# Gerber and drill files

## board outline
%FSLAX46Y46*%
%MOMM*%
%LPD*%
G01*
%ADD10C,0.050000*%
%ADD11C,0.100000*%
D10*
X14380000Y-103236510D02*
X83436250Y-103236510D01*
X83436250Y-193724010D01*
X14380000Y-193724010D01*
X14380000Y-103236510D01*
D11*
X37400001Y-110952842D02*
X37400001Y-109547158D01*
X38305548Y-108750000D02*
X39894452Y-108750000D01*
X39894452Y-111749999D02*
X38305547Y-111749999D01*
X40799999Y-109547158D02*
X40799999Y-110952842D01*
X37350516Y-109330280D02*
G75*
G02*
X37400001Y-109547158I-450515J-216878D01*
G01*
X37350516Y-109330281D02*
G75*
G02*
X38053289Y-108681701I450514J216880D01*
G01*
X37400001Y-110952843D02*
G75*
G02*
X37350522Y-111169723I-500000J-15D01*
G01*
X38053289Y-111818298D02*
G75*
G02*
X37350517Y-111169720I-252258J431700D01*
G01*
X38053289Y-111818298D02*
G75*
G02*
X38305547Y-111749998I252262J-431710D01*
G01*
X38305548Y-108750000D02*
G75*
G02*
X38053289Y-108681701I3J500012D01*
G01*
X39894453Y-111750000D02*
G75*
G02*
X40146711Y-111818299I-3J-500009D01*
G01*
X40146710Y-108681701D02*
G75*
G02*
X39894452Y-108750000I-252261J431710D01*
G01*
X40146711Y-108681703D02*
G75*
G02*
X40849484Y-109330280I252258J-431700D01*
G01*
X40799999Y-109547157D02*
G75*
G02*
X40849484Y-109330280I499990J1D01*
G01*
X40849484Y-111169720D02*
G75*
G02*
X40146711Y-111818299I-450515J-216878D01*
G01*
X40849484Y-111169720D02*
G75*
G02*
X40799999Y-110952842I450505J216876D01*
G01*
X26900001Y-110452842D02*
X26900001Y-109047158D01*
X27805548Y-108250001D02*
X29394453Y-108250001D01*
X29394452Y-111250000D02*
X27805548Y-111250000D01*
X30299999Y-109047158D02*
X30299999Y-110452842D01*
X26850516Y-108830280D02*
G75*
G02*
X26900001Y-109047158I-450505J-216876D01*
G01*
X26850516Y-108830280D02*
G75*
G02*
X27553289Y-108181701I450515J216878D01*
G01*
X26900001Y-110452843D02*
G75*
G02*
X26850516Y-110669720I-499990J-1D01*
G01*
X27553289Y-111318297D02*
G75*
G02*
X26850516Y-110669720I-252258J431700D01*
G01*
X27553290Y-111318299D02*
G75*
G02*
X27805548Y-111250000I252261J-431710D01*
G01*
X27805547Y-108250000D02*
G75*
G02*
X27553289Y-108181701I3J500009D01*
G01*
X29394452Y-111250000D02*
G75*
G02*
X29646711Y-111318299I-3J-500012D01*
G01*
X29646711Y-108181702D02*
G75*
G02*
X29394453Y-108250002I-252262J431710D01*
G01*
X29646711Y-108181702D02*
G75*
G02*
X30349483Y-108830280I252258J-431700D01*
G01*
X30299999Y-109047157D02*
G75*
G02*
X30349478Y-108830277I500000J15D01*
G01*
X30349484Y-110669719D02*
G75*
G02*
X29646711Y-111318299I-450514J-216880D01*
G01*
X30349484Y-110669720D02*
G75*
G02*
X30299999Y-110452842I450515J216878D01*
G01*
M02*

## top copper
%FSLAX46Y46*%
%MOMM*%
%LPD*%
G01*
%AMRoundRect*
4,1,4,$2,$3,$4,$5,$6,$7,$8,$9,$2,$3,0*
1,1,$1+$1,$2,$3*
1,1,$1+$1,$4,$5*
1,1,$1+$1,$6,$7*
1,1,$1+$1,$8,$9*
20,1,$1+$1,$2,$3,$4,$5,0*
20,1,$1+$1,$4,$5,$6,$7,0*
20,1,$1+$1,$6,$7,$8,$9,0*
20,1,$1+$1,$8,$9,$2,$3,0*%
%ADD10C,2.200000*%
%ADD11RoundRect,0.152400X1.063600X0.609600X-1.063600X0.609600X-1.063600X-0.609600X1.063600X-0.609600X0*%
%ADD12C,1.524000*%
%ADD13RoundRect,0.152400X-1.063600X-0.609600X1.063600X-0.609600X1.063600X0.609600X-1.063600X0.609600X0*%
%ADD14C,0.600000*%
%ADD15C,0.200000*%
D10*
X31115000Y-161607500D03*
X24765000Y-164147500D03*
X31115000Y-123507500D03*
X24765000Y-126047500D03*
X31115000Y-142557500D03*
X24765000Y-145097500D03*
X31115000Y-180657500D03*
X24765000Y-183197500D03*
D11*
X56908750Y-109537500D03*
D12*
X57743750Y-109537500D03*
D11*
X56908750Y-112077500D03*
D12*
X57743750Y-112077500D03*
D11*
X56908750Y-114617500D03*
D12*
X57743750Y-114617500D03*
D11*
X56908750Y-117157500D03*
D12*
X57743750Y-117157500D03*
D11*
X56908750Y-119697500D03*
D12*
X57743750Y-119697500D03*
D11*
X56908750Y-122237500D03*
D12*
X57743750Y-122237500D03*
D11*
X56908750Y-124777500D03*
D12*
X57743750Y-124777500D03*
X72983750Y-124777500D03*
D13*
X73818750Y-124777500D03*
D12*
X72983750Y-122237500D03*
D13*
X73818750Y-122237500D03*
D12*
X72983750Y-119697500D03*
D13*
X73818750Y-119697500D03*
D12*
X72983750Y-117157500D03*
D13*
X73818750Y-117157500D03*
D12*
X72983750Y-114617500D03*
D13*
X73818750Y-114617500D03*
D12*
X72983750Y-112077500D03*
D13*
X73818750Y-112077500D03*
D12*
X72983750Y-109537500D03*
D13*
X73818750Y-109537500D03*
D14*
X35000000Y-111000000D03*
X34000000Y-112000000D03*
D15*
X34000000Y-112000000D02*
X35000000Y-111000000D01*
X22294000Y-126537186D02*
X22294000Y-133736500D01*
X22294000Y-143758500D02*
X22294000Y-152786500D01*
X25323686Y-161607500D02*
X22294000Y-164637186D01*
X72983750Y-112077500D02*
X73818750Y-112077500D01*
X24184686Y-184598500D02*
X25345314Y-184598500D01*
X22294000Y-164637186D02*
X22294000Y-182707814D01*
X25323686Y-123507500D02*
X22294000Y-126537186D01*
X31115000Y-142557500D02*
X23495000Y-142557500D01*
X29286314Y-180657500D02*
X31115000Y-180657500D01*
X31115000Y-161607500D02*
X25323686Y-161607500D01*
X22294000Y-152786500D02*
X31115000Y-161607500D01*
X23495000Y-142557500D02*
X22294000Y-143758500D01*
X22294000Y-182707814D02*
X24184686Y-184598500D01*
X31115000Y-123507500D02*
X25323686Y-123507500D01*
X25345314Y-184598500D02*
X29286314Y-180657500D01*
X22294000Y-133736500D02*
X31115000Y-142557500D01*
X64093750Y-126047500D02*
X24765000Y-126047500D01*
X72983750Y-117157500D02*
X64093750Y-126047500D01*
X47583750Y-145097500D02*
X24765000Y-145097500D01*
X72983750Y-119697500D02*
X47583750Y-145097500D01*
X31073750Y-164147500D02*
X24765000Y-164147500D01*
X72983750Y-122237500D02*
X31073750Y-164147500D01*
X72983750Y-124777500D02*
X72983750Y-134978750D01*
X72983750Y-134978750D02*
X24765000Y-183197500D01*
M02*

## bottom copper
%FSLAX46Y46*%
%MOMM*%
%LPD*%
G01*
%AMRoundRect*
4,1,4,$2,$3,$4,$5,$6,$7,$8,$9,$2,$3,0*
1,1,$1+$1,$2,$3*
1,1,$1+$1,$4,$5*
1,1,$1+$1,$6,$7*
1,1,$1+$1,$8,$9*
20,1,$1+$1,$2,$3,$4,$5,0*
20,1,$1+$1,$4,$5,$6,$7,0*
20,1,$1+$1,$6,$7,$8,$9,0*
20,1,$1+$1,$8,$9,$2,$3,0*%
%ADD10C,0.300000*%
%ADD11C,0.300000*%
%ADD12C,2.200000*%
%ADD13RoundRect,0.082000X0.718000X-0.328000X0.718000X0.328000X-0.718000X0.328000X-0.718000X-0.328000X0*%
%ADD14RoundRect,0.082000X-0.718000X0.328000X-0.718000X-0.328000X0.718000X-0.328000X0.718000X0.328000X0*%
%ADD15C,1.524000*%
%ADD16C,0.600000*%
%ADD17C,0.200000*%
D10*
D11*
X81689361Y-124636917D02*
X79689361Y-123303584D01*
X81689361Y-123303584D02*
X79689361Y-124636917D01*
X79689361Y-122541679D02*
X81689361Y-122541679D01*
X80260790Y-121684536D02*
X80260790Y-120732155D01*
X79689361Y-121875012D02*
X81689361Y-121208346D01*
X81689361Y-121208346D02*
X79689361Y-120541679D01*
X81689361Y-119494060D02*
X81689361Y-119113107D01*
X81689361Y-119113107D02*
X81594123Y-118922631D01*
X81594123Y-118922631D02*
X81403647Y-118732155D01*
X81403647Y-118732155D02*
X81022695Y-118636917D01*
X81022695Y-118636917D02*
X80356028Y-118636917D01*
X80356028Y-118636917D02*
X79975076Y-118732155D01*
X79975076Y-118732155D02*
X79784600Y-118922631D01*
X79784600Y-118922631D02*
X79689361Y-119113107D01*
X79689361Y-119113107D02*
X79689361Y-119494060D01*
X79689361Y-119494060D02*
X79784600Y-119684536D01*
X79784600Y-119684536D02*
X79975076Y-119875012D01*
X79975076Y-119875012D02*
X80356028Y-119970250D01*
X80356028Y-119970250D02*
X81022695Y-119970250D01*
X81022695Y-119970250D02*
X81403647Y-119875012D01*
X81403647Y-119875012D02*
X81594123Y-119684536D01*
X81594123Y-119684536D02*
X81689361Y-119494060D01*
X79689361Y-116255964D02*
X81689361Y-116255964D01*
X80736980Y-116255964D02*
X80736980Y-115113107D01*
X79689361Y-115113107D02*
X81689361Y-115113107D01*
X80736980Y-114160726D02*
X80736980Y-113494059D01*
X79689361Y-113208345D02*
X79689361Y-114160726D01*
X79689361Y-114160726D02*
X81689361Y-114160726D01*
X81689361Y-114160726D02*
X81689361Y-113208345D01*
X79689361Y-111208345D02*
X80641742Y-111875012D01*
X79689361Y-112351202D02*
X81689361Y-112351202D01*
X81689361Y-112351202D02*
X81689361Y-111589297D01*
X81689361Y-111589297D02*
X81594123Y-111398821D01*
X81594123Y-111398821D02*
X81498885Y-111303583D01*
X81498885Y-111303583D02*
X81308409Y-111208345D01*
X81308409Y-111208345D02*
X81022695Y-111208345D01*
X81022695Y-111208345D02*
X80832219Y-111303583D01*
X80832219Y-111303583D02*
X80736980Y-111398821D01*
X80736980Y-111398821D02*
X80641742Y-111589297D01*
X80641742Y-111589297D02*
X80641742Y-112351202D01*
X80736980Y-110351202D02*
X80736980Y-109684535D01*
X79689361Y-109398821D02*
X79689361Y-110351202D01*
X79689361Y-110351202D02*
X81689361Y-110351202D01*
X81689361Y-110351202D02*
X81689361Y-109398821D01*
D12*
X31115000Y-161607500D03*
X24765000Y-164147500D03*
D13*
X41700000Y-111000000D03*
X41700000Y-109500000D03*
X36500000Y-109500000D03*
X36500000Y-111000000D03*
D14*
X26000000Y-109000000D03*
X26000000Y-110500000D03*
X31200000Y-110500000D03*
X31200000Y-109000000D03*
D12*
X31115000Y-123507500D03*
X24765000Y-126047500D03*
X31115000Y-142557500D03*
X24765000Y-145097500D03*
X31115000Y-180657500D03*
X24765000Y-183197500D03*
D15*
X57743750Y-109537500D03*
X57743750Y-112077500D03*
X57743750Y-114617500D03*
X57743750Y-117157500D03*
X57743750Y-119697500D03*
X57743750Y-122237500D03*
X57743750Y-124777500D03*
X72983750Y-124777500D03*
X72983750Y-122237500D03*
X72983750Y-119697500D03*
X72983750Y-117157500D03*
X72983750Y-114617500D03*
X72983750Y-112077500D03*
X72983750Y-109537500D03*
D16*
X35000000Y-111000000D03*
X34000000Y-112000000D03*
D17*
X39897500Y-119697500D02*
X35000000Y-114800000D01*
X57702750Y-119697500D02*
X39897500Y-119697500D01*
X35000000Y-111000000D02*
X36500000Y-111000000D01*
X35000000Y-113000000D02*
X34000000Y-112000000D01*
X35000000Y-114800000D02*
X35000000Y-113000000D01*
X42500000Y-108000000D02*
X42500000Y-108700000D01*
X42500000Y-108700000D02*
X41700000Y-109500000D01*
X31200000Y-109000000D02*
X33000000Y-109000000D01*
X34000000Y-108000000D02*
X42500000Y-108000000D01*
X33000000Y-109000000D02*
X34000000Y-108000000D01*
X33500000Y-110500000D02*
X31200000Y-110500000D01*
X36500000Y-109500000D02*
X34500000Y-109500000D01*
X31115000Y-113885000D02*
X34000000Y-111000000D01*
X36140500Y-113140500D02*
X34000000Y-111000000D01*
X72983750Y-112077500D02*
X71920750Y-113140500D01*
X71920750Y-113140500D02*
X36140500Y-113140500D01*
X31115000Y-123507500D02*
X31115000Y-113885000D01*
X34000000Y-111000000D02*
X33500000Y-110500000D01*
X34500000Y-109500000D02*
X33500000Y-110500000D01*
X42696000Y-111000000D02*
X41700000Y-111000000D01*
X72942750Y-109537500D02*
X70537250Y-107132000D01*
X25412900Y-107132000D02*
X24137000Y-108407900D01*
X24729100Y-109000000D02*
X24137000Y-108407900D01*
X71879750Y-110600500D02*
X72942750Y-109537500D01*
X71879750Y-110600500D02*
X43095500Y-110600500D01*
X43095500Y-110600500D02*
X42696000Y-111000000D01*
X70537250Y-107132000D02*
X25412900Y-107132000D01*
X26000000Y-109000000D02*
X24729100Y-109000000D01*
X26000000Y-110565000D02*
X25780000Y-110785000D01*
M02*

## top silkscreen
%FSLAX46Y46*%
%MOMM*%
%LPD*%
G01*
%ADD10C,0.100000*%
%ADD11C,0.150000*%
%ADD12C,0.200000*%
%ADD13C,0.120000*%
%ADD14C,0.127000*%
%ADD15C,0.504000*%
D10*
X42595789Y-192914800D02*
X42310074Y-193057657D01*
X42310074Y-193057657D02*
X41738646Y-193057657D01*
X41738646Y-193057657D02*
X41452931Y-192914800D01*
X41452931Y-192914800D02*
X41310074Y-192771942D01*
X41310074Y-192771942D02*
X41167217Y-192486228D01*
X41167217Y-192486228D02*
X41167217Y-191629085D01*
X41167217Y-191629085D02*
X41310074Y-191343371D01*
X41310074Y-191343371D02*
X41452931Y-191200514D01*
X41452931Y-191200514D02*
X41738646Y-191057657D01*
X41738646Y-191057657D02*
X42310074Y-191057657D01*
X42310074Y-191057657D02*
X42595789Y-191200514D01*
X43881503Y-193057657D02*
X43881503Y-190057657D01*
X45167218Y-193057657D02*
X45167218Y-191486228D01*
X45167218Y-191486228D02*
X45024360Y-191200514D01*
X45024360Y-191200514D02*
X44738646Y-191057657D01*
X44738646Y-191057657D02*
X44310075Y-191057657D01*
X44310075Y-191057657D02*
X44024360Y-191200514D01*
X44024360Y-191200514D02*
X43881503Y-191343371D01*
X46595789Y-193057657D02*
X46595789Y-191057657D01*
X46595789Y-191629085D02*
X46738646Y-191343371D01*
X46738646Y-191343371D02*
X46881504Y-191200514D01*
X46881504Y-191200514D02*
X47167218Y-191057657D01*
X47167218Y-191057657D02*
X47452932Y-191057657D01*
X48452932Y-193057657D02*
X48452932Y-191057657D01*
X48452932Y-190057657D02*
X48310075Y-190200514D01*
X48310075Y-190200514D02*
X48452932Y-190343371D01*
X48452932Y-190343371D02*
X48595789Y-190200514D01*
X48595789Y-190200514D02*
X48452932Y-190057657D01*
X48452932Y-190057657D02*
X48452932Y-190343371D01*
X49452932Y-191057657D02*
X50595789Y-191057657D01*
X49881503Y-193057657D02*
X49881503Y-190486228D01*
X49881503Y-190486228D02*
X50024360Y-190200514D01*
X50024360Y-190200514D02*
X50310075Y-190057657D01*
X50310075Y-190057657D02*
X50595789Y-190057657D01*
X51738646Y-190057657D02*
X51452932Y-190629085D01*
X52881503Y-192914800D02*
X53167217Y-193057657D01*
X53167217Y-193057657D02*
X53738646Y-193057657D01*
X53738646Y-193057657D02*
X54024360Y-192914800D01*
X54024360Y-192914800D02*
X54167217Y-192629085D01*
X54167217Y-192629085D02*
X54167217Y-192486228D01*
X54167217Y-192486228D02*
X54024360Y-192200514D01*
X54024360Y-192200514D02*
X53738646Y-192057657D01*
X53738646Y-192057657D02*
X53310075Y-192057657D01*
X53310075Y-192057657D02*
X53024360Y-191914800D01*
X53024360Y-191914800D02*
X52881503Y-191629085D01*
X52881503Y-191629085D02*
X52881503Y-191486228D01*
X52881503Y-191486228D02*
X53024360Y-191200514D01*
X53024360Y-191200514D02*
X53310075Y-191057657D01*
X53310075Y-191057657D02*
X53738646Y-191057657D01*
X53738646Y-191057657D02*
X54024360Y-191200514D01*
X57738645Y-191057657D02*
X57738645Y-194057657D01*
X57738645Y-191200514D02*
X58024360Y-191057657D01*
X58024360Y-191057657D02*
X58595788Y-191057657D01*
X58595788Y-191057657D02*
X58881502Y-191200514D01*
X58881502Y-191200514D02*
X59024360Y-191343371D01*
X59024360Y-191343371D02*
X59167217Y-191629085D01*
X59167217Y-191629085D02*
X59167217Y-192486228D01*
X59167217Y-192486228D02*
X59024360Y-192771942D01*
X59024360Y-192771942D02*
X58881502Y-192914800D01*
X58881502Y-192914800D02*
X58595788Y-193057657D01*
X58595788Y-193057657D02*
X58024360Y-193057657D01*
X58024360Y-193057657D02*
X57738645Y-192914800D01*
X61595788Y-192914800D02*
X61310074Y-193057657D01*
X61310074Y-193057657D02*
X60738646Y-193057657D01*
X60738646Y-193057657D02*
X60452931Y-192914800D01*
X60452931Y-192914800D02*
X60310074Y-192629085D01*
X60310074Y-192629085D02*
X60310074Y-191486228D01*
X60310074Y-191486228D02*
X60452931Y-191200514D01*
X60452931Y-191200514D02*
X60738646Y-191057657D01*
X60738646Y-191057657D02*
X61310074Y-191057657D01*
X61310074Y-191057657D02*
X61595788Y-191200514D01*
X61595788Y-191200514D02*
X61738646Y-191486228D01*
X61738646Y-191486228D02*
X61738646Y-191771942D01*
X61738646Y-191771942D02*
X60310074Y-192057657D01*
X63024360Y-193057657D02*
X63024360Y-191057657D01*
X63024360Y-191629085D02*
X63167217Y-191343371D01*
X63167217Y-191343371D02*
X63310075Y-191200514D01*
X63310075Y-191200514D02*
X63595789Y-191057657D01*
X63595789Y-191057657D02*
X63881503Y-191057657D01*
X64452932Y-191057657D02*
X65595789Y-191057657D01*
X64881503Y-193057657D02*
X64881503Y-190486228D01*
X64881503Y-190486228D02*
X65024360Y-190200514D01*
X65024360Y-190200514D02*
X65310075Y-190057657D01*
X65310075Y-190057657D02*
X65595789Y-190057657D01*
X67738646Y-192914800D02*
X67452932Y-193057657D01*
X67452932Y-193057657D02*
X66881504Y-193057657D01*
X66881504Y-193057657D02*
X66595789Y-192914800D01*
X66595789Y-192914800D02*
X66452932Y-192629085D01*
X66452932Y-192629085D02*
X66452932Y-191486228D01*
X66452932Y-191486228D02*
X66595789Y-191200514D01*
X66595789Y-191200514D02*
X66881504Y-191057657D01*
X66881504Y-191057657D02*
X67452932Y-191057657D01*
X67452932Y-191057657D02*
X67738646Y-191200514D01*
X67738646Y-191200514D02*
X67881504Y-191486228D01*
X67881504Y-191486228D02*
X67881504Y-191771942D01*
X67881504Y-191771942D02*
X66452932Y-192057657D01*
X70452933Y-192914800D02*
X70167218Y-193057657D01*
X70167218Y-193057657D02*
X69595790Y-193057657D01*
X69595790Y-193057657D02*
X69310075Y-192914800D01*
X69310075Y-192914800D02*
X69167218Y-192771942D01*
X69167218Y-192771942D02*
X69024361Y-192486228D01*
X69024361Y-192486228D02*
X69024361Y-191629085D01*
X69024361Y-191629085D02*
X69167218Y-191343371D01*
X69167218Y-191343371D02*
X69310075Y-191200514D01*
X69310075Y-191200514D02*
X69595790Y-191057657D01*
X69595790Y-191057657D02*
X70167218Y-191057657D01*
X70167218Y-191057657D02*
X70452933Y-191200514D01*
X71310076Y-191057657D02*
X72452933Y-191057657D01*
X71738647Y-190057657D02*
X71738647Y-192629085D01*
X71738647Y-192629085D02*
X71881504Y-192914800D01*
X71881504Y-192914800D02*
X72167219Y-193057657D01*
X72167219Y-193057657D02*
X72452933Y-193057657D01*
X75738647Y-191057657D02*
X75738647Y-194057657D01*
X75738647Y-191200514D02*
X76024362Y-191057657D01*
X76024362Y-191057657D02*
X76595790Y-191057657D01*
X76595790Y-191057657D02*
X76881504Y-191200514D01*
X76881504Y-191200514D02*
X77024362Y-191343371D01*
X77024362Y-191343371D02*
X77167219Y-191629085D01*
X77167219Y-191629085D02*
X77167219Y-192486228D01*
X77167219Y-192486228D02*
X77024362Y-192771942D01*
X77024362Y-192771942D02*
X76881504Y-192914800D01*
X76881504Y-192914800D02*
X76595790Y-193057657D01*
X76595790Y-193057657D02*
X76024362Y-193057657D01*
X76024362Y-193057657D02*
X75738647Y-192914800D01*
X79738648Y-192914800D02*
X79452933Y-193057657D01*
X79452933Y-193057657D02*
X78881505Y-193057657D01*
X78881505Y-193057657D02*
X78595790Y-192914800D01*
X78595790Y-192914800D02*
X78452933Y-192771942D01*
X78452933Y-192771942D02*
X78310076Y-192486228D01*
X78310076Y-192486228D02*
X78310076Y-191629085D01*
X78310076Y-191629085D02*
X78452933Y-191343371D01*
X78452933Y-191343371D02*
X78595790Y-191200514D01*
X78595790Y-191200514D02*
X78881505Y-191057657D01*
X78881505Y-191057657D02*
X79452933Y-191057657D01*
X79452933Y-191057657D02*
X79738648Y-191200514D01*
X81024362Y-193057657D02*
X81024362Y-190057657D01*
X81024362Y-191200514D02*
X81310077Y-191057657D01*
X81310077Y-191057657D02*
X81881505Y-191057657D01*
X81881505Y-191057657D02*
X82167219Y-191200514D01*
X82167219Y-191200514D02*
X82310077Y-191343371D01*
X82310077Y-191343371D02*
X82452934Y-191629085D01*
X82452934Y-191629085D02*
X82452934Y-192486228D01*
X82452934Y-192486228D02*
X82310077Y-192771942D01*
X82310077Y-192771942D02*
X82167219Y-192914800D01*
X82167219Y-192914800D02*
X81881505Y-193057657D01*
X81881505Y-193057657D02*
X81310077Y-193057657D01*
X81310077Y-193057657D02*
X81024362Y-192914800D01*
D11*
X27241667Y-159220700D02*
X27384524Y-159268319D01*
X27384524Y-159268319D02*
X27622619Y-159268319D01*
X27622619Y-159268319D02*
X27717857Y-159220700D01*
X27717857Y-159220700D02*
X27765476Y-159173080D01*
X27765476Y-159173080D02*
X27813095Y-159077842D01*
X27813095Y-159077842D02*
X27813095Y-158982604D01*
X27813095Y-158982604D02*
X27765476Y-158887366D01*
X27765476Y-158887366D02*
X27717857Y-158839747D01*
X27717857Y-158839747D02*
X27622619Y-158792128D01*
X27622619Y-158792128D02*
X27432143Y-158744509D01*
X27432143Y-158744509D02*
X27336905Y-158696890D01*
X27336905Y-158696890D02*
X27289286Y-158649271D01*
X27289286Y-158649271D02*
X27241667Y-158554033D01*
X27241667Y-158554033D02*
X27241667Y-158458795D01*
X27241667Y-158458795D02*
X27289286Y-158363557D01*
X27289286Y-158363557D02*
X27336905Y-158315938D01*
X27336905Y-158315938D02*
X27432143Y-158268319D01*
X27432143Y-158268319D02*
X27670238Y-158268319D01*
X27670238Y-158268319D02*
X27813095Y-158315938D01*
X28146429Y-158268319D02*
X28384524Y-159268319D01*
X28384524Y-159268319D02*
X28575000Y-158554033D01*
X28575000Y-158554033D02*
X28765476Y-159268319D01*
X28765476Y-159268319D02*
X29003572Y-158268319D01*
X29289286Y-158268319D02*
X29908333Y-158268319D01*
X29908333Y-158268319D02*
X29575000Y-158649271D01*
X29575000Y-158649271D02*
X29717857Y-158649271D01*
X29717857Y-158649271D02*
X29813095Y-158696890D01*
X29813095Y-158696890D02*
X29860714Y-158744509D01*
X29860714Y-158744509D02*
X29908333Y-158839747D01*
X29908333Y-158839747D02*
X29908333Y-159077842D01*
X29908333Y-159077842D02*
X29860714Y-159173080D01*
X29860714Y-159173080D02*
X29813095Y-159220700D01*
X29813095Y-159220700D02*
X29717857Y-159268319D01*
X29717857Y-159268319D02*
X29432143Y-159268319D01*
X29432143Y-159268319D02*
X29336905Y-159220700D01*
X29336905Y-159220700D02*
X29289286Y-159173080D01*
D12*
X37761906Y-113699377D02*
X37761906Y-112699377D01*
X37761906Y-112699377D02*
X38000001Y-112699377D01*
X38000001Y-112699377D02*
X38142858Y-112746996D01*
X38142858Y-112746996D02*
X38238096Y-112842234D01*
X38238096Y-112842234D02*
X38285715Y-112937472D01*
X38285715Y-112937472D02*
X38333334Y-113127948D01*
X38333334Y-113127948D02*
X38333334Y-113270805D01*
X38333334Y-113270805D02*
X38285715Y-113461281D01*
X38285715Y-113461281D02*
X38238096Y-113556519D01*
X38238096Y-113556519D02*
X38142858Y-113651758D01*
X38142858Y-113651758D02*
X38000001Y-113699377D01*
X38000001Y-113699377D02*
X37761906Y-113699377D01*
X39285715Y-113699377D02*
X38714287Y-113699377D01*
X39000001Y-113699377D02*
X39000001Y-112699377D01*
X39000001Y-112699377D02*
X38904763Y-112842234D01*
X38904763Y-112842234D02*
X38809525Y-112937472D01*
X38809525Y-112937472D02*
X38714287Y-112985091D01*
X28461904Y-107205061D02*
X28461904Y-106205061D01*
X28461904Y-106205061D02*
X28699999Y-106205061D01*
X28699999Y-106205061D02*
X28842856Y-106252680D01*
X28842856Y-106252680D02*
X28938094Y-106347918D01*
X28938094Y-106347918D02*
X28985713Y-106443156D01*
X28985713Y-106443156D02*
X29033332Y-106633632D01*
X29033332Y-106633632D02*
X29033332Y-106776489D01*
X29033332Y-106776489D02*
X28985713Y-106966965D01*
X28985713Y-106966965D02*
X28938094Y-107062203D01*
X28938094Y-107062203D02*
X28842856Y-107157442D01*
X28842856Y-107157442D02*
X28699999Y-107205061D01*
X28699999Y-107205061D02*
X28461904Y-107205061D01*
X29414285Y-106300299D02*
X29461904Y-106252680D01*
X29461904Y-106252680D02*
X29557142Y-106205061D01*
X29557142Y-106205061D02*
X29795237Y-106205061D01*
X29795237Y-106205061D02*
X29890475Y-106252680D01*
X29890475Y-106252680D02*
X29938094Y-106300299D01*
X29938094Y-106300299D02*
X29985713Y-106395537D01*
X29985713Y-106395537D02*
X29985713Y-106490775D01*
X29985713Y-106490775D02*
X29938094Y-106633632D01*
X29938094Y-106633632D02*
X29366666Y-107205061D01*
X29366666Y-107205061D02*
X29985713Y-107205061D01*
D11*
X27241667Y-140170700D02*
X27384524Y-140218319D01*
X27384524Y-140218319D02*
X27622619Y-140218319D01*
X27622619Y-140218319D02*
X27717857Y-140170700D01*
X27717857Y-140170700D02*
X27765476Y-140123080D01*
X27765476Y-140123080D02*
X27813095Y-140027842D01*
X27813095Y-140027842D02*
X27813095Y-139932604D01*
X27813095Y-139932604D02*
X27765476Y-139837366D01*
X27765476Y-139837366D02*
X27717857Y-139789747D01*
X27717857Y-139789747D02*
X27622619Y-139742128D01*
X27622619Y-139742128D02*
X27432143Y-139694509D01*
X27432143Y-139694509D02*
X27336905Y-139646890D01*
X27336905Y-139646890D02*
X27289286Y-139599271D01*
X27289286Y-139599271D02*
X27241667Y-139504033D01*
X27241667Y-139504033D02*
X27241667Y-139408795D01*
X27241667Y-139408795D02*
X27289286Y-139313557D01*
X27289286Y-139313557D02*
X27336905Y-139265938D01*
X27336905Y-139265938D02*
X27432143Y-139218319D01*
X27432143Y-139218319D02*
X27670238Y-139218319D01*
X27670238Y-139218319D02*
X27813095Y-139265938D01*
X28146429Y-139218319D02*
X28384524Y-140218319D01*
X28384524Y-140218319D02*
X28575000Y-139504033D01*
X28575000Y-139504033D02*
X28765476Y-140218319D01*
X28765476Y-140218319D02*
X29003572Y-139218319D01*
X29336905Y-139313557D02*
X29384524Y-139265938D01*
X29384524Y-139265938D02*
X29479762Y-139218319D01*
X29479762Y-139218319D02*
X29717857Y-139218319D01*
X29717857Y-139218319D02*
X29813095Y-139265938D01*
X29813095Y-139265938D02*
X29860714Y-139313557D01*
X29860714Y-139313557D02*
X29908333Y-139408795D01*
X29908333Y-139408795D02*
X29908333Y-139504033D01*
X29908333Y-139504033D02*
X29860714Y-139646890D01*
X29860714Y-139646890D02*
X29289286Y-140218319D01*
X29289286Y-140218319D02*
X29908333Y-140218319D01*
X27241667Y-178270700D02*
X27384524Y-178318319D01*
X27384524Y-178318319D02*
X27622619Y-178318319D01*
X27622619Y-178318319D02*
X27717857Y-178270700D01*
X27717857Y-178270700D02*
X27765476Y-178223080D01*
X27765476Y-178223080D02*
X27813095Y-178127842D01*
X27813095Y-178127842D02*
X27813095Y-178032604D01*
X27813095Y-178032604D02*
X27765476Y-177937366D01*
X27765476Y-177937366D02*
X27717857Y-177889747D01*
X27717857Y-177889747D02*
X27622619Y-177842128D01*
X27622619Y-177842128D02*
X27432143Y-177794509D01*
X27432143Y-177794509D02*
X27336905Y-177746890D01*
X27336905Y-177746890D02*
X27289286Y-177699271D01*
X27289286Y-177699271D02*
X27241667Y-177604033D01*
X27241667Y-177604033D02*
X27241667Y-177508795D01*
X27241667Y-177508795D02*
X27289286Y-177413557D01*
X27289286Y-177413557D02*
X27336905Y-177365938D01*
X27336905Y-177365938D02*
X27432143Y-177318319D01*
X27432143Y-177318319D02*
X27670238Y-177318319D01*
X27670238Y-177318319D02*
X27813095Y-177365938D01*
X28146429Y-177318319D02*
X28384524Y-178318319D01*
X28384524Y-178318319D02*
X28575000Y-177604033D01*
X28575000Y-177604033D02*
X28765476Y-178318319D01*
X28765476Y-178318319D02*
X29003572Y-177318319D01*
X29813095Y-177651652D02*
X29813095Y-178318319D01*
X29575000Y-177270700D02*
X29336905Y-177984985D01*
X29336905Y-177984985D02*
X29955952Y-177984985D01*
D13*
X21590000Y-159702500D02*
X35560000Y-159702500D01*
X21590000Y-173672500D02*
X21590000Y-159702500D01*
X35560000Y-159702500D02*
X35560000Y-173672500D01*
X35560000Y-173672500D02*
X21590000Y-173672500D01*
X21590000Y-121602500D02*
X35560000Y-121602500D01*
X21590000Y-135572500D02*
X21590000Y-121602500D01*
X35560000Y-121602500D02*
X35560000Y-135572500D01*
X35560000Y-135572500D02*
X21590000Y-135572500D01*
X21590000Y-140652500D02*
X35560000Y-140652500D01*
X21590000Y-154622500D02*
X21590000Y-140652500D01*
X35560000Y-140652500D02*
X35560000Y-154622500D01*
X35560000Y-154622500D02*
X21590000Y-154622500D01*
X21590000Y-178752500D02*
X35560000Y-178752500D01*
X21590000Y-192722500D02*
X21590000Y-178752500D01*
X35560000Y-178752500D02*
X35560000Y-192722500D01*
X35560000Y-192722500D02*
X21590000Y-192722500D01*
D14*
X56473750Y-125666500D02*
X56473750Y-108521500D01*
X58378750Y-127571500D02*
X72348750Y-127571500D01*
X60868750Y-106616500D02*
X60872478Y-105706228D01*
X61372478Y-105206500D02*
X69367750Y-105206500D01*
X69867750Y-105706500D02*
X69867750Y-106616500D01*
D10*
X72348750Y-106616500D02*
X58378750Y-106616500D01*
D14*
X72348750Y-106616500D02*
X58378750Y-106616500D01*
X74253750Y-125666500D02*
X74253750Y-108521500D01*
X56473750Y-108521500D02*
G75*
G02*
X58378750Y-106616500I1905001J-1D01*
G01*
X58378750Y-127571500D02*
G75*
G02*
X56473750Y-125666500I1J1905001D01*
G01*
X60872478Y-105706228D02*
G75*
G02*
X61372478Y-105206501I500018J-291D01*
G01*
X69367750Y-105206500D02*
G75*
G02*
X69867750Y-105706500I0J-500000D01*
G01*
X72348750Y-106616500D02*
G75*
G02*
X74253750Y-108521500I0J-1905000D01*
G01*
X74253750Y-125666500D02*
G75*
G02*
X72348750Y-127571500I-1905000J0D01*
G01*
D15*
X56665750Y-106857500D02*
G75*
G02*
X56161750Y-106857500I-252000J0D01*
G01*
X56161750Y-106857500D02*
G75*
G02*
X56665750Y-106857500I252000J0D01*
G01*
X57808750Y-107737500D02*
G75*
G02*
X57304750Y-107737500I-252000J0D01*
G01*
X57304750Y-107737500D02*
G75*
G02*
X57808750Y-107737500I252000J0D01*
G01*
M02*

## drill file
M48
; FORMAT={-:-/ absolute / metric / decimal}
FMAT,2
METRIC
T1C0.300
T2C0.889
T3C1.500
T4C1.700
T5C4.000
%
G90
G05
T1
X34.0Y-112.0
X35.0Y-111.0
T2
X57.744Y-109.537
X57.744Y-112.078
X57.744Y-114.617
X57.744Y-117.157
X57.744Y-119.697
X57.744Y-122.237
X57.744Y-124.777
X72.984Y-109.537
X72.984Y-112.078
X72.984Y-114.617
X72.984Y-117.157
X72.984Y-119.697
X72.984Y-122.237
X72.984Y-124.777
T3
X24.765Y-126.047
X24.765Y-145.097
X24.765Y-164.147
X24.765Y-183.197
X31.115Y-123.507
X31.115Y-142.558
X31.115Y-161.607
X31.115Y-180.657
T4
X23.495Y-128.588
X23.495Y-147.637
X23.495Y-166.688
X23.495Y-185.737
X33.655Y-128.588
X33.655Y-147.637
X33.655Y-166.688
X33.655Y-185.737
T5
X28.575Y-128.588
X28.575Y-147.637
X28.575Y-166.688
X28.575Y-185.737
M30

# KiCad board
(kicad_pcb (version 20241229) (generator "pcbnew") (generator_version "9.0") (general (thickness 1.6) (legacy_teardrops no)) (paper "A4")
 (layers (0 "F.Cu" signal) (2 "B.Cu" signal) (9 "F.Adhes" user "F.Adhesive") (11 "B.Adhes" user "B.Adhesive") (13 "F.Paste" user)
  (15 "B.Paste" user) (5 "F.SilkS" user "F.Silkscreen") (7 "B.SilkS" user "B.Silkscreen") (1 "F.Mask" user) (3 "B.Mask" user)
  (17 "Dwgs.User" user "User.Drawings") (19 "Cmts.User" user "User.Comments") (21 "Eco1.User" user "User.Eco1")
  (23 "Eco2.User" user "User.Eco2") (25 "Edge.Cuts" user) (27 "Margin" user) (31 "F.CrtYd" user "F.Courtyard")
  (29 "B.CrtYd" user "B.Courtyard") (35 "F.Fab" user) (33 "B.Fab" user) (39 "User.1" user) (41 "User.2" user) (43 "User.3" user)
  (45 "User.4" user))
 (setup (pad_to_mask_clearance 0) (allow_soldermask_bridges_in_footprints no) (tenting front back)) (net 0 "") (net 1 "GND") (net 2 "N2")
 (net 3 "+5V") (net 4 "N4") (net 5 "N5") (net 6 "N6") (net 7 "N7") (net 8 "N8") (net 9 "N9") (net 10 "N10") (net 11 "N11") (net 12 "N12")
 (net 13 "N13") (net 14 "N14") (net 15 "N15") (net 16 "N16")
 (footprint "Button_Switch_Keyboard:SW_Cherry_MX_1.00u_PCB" (layer "F.Cu") (at 31.115 161.6075)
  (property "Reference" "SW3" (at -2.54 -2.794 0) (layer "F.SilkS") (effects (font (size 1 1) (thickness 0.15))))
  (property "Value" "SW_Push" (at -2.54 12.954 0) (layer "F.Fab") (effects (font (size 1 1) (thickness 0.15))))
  (fp_line (start -9.525 -1.905) (end 4.445 -1.905) (stroke (width 0.12) (type solid)) (layer "F.SilkS"))
  (fp_line (start -9.525 12.065) (end -9.525 -1.905) (stroke (width 0.12) (type solid)) (layer "F.SilkS"))
  (fp_line (start 4.445 -1.905) (end 4.445 12.065) (stroke (width 0.12) (type solid)) (layer "F.SilkS"))
  (fp_line (start 4.445 12.065) (end -9.525 12.065) (stroke (width 0.12) (type solid)) (layer "F.SilkS"))
  (pad "" np_thru_hole circle (at -7.62 5.08) (size 1.7 1.7) (drill 1.7) (layers "*.Cu" "*.Mask"))
  (pad "" np_thru_hole circle (at -2.54 5.08) (size 4 4) (drill 4) (layers "*.Cu" "*.Mask"))
  (pad "" np_thru_hole circle (at 2.54 5.08) (size 1.7 1.7) (drill 1.7) (layers "*.Cu" "*.Mask"))
  (pad "1" thru_hole circle (at 0 0) (size 2.2 2.2) (drill 1.5) (layers "*.Cu" "*.Mask") (remove_unused_layers no) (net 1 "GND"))
  (pad "2" thru_hole circle (at -6.35 2.54) (size 2.2 2.2) (drill 1.5) (layers "*.Cu" "*.Mask") (remove_unused_layers no) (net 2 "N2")))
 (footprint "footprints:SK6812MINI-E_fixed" (layer "F.Cu") (at 39.100001 110.147158 180)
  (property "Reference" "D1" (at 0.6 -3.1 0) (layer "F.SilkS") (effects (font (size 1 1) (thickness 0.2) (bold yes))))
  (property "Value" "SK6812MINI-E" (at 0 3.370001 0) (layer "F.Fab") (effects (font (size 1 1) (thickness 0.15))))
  (fp_line (start 1.7 -0.805684) (end 1.7 0.6) (stroke (width 0.1) (type solid)) (layer "Edge.Cuts"))
  (fp_line (start 0.794453 1.397158) (end -0.794451 1.397158) (stroke (width 0.1) (type solid)) (layer "Edge.Cuts"))
  (fp_line (start -0.794451 -1.602841) (end 0.794454 -1.602841) (stroke (width 0.1) (type solid)) (layer "Edge.Cuts"))
  (fp_line (start -1.699998 0.6) (end -1.699998 -0.805684) (stroke (width 0.1) (type solid)) (layer "Edge.Cuts"))
  (fp_arc (start 1.749485 0.816878) (mid 1.712528 0.711226) (end 1.7 0.6) (stroke (width 0.1) (type solid)) (layer "Edge.Cuts"))
  (fp_arc (start 1.749485 0.816877) (mid 1.638073 1.401193) (end 1.046712 1.465457) (stroke (width 0.1) (type solid)) (layer "Edge.Cuts"))
  (fp_arc (start 1.7 -0.805685) (mid 1.712528 -0.91691) (end 1.749485 -1.022562) (stroke (width 0.1) (type solid)) (layer "Edge.Cuts"))
  (fp_arc (start 1.046712 -1.67114) (mid 1.638072 -1.606876) (end 1.749485 -1.022562) (stroke (width 0.1) (type solid)) (layer "Edge.Cuts"))
  (fp_arc (start 1.046712 -1.67114) (mid 0.925124 -1.620218) (end 0.794454 -1.602841) (stroke (width 0.1) (type solid)) (layer "Edge.Cuts"))
  (fp_arc (start 0.794453 1.397158) (mid 0.925124 1.414535) (end 1.046712 1.465457) (stroke (width 0.1) (type solid)) (layer "Edge.Cuts"))
  (fp_arc (start -0.794452 -1.602842) (mid -0.925122 -1.620219) (end -1.04671 -1.671141) (stroke (width 0.1) (type solid))
   (layer "Edge.Cuts"))
  (fp_arc (start -1.046709 1.465457) (mid -0.925121 1.414535) (end -0.794451 1.397158) (stroke (width 0.1) (type solid)) (layer "Edge.Cuts"))
  (fp_arc (start -1.04671 1.465455) (mid -1.638069 1.401192) (end -1.749483 0.816878) (stroke (width 0.1) (type solid)) (layer "Edge.Cuts"))
  (fp_arc (start -1.699998 0.600001) (mid -1.712526 0.711226) (end -1.749483 0.816878) (stroke (width 0.1) (type solid)) (layer "Edge.Cuts"))
  (fp_arc (start -1.749483 -1.022562) (mid -1.63807 -1.606877) (end -1.04671 -1.671141) (stroke (width 0.1) (type solid))
   (layer "Edge.Cuts"))
  (fp_arc (start -1.749483 -1.022562) (mid -1.712526 -0.91691) (end -1.699998 -0.805684) (stroke (width 0.1) (type solid))
   (layer "Edge.Cuts"))
  (pad "1" smd roundrect (at -2.599999 -0.852842 90) (size 0.82 1.6) (layers "B.Cu" "B.Mask" "B.Paste") (roundrect_rratio 0.1) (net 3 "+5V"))
  (pad "2" smd roundrect (at -2.599999 0.647158 90) (size 0.82 1.6) (layers "B.Cu" "B.Mask" "B.Paste") (roundrect_rratio 0.1) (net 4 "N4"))
  (pad "3" smd roundrect (at 2.600001 0.647158 90) (size 0.82 1.6) (layers "B.Cu" "B.Mask" "B.Paste") (roundrect_rratio 0.1) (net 1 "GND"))
  (pad "4" smd roundrect (at 2.600001 -0.852842 90) (size 0.82 1.6) (layers "B.Cu" "B.Mask" "B.Paste") (roundrect_rratio 0.1) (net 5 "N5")))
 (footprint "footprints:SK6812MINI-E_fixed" (layer "F.Cu") (at 28.599999 109.852842)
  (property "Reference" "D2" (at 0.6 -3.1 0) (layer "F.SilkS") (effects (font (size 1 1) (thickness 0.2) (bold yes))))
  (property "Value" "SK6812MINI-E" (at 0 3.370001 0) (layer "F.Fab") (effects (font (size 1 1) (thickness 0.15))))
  (fp_line (start -1.699998 0.6) (end -1.699998 -0.805684) (stroke (width 0.1) (type solid)) (layer "Edge.Cuts"))
  (fp_line (start -0.794451 -1.602841) (end 0.794454 -1.602841) (stroke (width 0.1) (type solid)) (layer "Edge.Cuts"))
  (fp_line (start 0.794453 1.397158) (end -0.794451 1.397158) (stroke (width 0.1) (type solid)) (layer "Edge.Cuts"))
  (fp_line (start 1.7 -0.805684) (end 1.7 0.6) (stroke (width 0.1) (type solid)) (layer "Edge.Cuts"))
  (fp_arc (start -1.749483 -1.022562) (mid -1.712526 -0.91691) (end -1.699998 -0.805684) (stroke (width 0.1) (type solid))
   (layer "Edge.Cuts"))
  (fp_arc (start -1.749483 -1.022562) (mid -1.63807 -1.606877) (end -1.04671 -1.671141) (stroke (width 0.1) (type solid))
   (layer "Edge.Cuts"))
  (fp_arc (start -1.699998 0.600001) (mid -1.712526 0.711226) (end -1.749483 0.816878) (stroke (width 0.1) (type solid)) (layer "Edge.Cuts"))
  (fp_arc (start -1.04671 1.465455) (mid -1.638069 1.401192) (end -1.749483 0.816878) (stroke (width 0.1) (type solid)) (layer "Edge.Cuts"))
  (fp_arc (start -1.046709 1.465457) (mid -0.925121 1.414535) (end -0.794451 1.397158) (stroke (width 0.1) (type solid)) (layer "Edge.Cuts"))
  (fp_arc (start -0.794452 -1.602842) (mid -0.925122 -1.620219) (end -1.04671 -1.671141) (stroke (width 0.1) (type solid))
   (layer "Edge.Cuts"))
  (fp_arc (start 0.794453 1.397158) (mid 0.925124 1.414535) (end 1.046712 1.465457) (stroke (width 0.1) (type solid)) (layer "Edge.Cuts"))
  (fp_arc (start 1.046712 -1.67114) (mid 0.925124 -1.620218) (end 0.794454 -1.602841) (stroke (width 0.1) (type solid)) (layer "Edge.Cuts"))
  (fp_arc (start 1.046712 -1.67114) (mid 1.638072 -1.606876) (end 1.749485 -1.022562) (stroke (width 0.1) (type solid)) (layer "Edge.Cuts"))
  (fp_arc (start 1.7 -0.805685) (mid 1.712528 -0.91691) (end 1.749485 -1.022562) (stroke (width 0.1) (type solid)) (layer "Edge.Cuts"))
  (fp_arc (start 1.749485 0.816877) (mid 1.638073 1.401193) (end 1.046712 1.465457) (stroke (width 0.1) (type solid)) (layer "Edge.Cuts"))
  (fp_arc (start 1.749485 0.816878) (mid 1.712528 0.711226) (end 1.7 0.6) (stroke (width 0.1) (type solid)) (layer "Edge.Cuts"))
  (pad "1" smd roundrect (at -2.599999 -0.852842 270) (size 0.82 1.6) (layers "B.Cu" "B.Mask" "B.Paste") (roundrect_rratio 0.1)
   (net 3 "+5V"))
  (pad "2" smd roundrect (at -2.599999 0.647158 270) (size 0.82 1.6) (layers "B.Cu" "B.Mask" "B.Paste") (roundrect_rratio 0.1) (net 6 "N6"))
  (pad "3" smd roundrect (at 2.600001 0.647158 270) (size 0.82 1.6) (layers "B.Cu" "B.Mask" "B.Paste") (roundrect_rratio 0.1) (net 1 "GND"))
  (pad "4" smd roundrect (at 2.600001 -0.852842 270) (size 0.82 1.6) (layers "B.Cu" "B.Mask" "B.Paste") (roundrect_rratio 0.1) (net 4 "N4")))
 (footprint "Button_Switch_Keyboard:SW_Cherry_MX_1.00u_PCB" (layer "F.Cu") (at 31.115 123.5075)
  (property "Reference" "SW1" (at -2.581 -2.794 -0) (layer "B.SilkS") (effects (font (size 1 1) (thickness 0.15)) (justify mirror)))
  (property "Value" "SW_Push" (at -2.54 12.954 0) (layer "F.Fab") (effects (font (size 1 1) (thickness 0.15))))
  (fp_line (start -9.525 -1.905) (end 4.445 -1.905) (stroke (width 0.12) (type solid)) (layer "F.SilkS"))
  (fp_line (start -9.525 12.065) (end -9.525 -1.905) (stroke (width 0.12) (type solid)) (layer "F.SilkS"))
  (fp_line (start 4.445 -1.905) (end 4.445 12.065) (stroke (width 0.12) (type solid)) (layer "F.SilkS"))
  (fp_line (start 4.445 12.065) (end -9.525 12.065) (stroke (width 0.12) (type solid)) (layer "F.SilkS"))
  (pad "" np_thru_hole circle (at -7.62 5.08) (size 1.7 1.7) (drill 1.7) (layers "*.Cu" "*.Mask"))
  (pad "" np_thru_hole circle (at -2.54 5.08) (size 4 4) (drill 4) (layers "*.Cu" "*.Mask"))
  (pad "" np_thru_hole circle (at 2.54 5.08) (size 1.7 1.7) (drill 1.7) (layers "*.Cu" "*.Mask"))
  (pad "1" thru_hole circle (at 0 0) (size 2.2 2.2) (drill 1.5) (layers "*.Cu" "*.Mask") (remove_unused_layers no) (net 1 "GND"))
  (pad "2" thru_hole circle (at -6.35 2.54) (size 2.2 2.2) (drill 1.5) (layers "*.Cu" "*.Mask") (remove_unused_layers no) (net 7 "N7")))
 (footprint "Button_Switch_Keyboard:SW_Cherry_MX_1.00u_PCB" (layer "F.Cu") (at 31.115 142.5575)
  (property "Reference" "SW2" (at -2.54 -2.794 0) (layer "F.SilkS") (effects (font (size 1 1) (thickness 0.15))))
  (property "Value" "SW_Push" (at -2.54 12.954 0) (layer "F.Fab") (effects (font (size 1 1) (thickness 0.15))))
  (fp_line (start -9.525 -1.905) (end 4.445 -1.905) (stroke (width 0.12) (type solid)) (layer "F.SilkS"))
  (fp_line (start -9.525 12.065) (end -9.525 -1.905) (stroke (width 0.12) (type solid)) (layer "F.SilkS"))
  (fp_line (start 4.445 -1.905) (end 4.445 12.065) (stroke (width 0.12) (type solid)) (layer "F.SilkS"))
  (fp_line (start 4.445 12.065) (end -9.525 12.065) (stroke (width 0.12) (type solid)) (layer "F.SilkS"))
  (pad "" np_thru_hole circle (at -7.62 5.08) (size 1.7 1.7) (drill 1.7) (layers "*.Cu" "*.Mask"))
  (pad "" np_thru_hole circle (at -2.54 5.08) (size 4 4) (drill 4) (layers "*.Cu" "*.Mask"))
  (pad "" np_thru_hole circle (at 2.54 5.08) (size 1.7 1.7) (drill 1.7) (layers "*.Cu" "*.Mask"))
  (pad "1" thru_hole circle (at 0 0) (size 2.2 2.2) (drill 1.5) (layers "*.Cu" "*.Mask") (remove_unused_layers no) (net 1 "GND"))
  (pad "2" thru_hole circle (at -6.35 2.54) (size 2.2 2.2) (drill 1.5) (layers "*.Cu" "*.Mask") (remove_unused_layers no) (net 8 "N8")))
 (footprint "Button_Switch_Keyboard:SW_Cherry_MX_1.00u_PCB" (layer "F.Cu") (at 31.115 180.6575)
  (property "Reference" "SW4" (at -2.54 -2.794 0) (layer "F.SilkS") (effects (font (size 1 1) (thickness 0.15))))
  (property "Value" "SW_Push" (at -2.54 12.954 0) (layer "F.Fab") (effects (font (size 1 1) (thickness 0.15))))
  (fp_line (start -9.525 -1.905) (end 4.445 -1.905) (stroke (width 0.12) (type solid)) (layer "F.SilkS"))
  (fp_line (start -9.525 12.065) (end -9.525 -1.905) (stroke (width 0.12) (type solid)) (layer "F.SilkS"))
  (fp_line (start 4.445 -1.905) (end 4.445 12.065) (stroke (width 0.12) (type solid)) (layer "F.SilkS"))
  (fp_line (start 4.445 12.065) (end -9.525 12.065) (stroke (width 0.12) (type solid)) (layer "F.SilkS"))
  (pad "" np_thru_hole circle (at -7.62 5.08) (size 1.7 1.7) (drill 1.7) (layers "*.Cu" "*.Mask"))
  (pad "" np_thru_hole circle (at -2.54 5.08) (size 4 4) (drill 4) (layers "*.Cu" "*.Mask"))
  (pad "" np_thru_hole circle (at 2.54 5.08) (size 1.7 1.7) (drill 1.7) (layers "*.Cu" "*.Mask"))
  (pad "1" thru_hole circle (at 0 0) (size 2.2 2.2) (drill 1.5) (layers "*.Cu" "*.Mask") (remove_unused_layers no) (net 1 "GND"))
  (pad "2" thru_hole circle (at -6.35 2.54) (size 2.2 2.2) (drill 1.5) (layers "*.Cu" "*.Mask") (remove_unused_layers no) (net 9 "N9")))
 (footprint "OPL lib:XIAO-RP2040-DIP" (layer "F.Cu") (at 65.36375 117.1575)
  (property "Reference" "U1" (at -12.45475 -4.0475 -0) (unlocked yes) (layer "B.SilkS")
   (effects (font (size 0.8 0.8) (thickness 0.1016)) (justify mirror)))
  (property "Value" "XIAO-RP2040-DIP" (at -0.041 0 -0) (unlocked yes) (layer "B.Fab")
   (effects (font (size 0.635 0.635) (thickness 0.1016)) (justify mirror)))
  (fp_line (start -8.89 8.509) (end -8.89 -8.636) (stroke (width 0.127) (type solid)) (layer "F.SilkS"))
  (fp_line (start -6.985 10.414) (end 6.985 10.414) (stroke (width 0.127) (type solid)) (layer "F.SilkS"))
  (fp_line (start -4.495 -10.541) (end -4.491272 -11.451272) (stroke (width 0.127) (type solid)) (layer "F.SilkS"))
  (fp_line (start -3.991272 -11.951) (end 4.004 -11.951) (stroke (width 0.127) (type solid)) (layer "F.SilkS"))
  (fp_line (start 4.504 -11.451) (end 4.504 -10.541) (stroke (width 0.127) (type solid)) (layer "F.SilkS"))
  (fp_line (start 6.985 -10.541) (end -6.985 -10.541) (stroke (width 0.1) (type solid)) (layer "F.SilkS"))
  (fp_line (start 6.985 -10.541) (end -6.985 -10.541) (stroke (width 0.127) (type solid)) (layer "F.SilkS"))
  (fp_line (start 8.89 8.509) (end 8.89 -8.636) (stroke (width 0.127) (type solid)) (layer "F.SilkS"))
  (fp_arc (start -8.89 -8.636) (mid -8.332038 -9.983038) (end -6.985 -10.541) (stroke (width 0.127) (type solid)) (layer "F.SilkS"))
  (fp_arc (start -6.985 10.414) (mid -8.332038 9.856038) (end -8.89 8.509) (stroke (width 0.127) (type solid)) (layer "F.SilkS"))
  (fp_arc (start -4.491272 -11.451272) (mid -4.344728 -11.80464) (end -3.991272 -11.951) (stroke (width 0.127) (type default))
   (layer "F.SilkS"))
  (fp_arc (start 4.004 -11.951) (mid 4.357553 -11.804553) (end 4.504 -11.451) (stroke (width 0.127) (type default)) (layer "F.SilkS"))
  (fp_arc (start 6.985 -10.541) (mid 8.332038 -9.983038) (end 8.89 -8.636) (stroke (width 0.127) (type solid)) (layer "F.SilkS"))
  (fp_arc (start 8.89 8.509) (mid 8.332038 9.856038) (end 6.985 10.414) (stroke (width 0.127) (type solid)) (layer "F.SilkS"))
  (fp_circle (center -8.95 -10.3) (end -8.95 -10.554) (stroke (width 0.5) (type solid)) (fill yes) (layer "F.SilkS"))
  (fp_circle (center -7.807 -9.42) (end -7.807 -9.674) (stroke (width 0.5) (type solid)) (fill yes) (layer "F.SilkS"))
  (pad "1" smd roundrect (at -8.455 -7.62 180) (size 2.432 1.524) (layers "F.Cu" "F.Mask") (roundrect_rratio 0.1) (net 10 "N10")
   (thermal_bridge_angle 45))
  (pad "1" thru_hole circle (at -7.62 -7.62 180) (size 1.524 1.524) (drill 0.889) (layers "*.Cu" "*.Mask") (remove_unused_layers no)
   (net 10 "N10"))
  (pad "2" smd roundrect (at -8.455 -5.08 180) (size 2.432 1.524) (layers "F.Cu" "F.Mask") (roundrect_rratio 0.1) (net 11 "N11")
   (thermal_bridge_angle 45))
  (pad "2" thru_hole circle (at -7.62 -5.08 180) (size 1.524 1.524) (drill 0.889) (layers "*.Cu" "*.Mask") (remove_unused_layers no)
   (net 11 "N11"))
  (pad "3" smd roundrect (at -8.455 -2.54 180) (size 2.432 1.524) (layers "F.Cu" "F.Mask") (roundrect_rratio 0.1) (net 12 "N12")
   (thermal_bridge_angle 45))
  (pad "3" thru_hole circle (at -7.62 -2.54 180) (size 1.524 1.524) (drill 0.889) (layers "*.Cu" "*.Mask") (remove_unused_layers no)
   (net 12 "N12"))
  (pad "4" smd roundrect (at -8.455 0 180) (size 2.432 1.524) (layers "F.Cu" "F.Mask") (roundrect_rratio 0.1) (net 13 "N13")
   (thermal_bridge_angle 45))
  (pad "4" thru_hole circle (at -7.62 0 180) (size 1.524 1.524) (drill 0.889) (layers "*.Cu" "*.Mask") (remove_unused_layers no)
   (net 13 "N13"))
  (pad "5" smd roundrect (at -8.455 2.54 180) (size 2.432 1.524) (layers "F.Cu" "F.Mask") (roundrect_rratio 0.1) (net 5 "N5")
   (thermal_bridge_angle 45))
  (pad "5" thru_hole circle (at -7.62 2.54 180) (size 1.524 1.524) (drill 0.889) (layers "*.Cu" "*.Mask") (remove_unused_layers no)
   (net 5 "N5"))
  (pad "6" smd roundrect (at -8.455 5.08 180) (size 2.432 1.524) (layers "F.Cu" "F.Mask") (roundrect_rratio 0.1) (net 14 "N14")
   (thermal_bridge_angle 45))
  (pad "6" thru_hole circle (at -7.62 5.08 180) (size 1.524 1.524) (drill 0.889) (layers "*.Cu" "*.Mask") (remove_unused_layers no)
   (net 14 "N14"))
  (pad "7" smd roundrect (at -8.455 7.62 180) (size 2.432 1.524) (layers "F.Cu" "F.Mask") (roundrect_rratio 0.1) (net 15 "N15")
   (thermal_bridge_angle 45))
  (pad "7" thru_hole circle (at -7.62 7.62 180) (size 1.524 1.524) (drill 0.889) (layers "*.Cu" "*.Mask") (remove_unused_layers no)
   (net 15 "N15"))
  (pad "8" thru_hole circle (at 7.62 7.62) (size 1.524 1.524) (drill 0.889) (layers "*.Cu" "*.Mask") (remove_unused_layers no) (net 9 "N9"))
  (pad "8" smd roundrect (at 8.455 7.62) (size 2.432 1.524) (layers "F.Cu" "F.Mask") (roundrect_rratio 0.1) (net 9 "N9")
   (thermal_bridge_angle 45))
  (pad "9" thru_hole circle (at 7.62 5.08) (size 1.524 1.524) (drill 0.889) (layers "*.Cu" "*.Mask") (remove_unused_layers no) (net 2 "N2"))
  (pad "9" smd roundrect (at 8.455 5.08) (size 2.432 1.524) (layers "F.Cu" "F.Mask") (roundrect_rratio 0.1) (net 2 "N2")
   (thermal_bridge_angle 45))
  (pad "10" thru_hole circle (at 7.62 2.54) (size 1.524 1.524) (drill 0.889) (layers "*.Cu" "*.Mask") (remove_unused_layers no) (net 8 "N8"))
  (pad "10" smd roundrect (at 8.455 2.54) (size 2.432 1.524) (layers "F.Cu" "F.Mask") (roundrect_rratio 0.1) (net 8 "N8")
   (thermal_bridge_angle 45))
  (pad "11" thru_hole circle (at 7.62 0) (size 1.524 1.524) (drill 0.889) (layers "*.Cu" "*.Mask") (remove_unused_layers no) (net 7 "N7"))
  (pad "11" smd roundrect (at 8.455 0) (size 2.432 1.524) (layers "F.Cu" "F.Mask") (roundrect_rratio 0.1) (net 7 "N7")
   (thermal_bridge_angle 45))
  (pad "12" thru_hole circle (at 7.62 -2.54) (size 1.524 1.524) (drill 0.889) (layers "*.Cu" "*.Mask") (remove_unused_layers no)
   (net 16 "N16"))
  (pad "12" smd roundrect (at 8.455 -2.54) (size 2.432 1.524) (layers "F.Cu" "F.Mask") (roundrect_rratio 0.1) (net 16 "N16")
   (thermal_bridge_angle 45))
  (pad "13" thru_hole circle (at 7.62 -5.08) (size 1.524 1.524) (drill 0.889) (layers "*.Cu" "*.Mask") (remove_unused_layers no)
   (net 1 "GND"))
  (pad "13" smd roundrect (at 8.455 -5.08) (size 2.432 1.524) (layers "F.Cu" "F.Mask") (roundrect_rratio 0.1) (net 1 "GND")
   (thermal_bridge_angle 45))
  (pad "14" thru_hole circle (at 7.62 -7.62) (size 1.524 1.524) (drill 0.889) (layers "*.Cu" "*.Mask") (remove_unused_layers no)
   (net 3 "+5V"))
  (pad "14" smd roundrect (at 8.455 -7.62) (size 2.432 1.524) (layers "F.Cu" "F.Mask") (roundrect_rratio 0.1) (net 3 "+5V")
   (thermal_bridge_angle 45)))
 (gr_rect (start 14.38 103.23651) (end 83.43625 193.72401) (stroke (width 0.05) (type default)) (fill no) (layer "Edge.Cuts"))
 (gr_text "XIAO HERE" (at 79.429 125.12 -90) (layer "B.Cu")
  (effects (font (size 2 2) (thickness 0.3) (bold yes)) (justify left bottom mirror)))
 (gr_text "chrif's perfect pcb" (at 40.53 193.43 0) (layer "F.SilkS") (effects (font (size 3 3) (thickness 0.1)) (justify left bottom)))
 (segment (start 34 112) (end 35 111) (width 0.2) (layer "F.Cu") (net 5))
 (via (at 35 111) (size 0.6) (drill 0.3) (layers "F.Cu" "B.Cu") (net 5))
 (via (at 34 112) (size 0.6) (drill 0.3) (layers "F.Cu" "B.Cu") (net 5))
 (segment (start 39.8975 119.6975) (end 35 114.8) (width 0.2) (layer "B.Cu") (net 5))
 (segment (start 57.70275 119.6975) (end 39.8975 119.6975) (width 0.2) (layer "B.Cu") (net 5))
 (segment (start 35 111) (end 36.5 111) (width 0.2) (layer "B.Cu") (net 5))
 (segment (start 35 113) (end 34 112) (width 0.2) (layer "B.Cu") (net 5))
 (segment (start 35 114.8) (end 35 113) (width 0.2) (layer "B.Cu") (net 5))
 (segment (start 42.5 108) (end 42.5 108.7) (width 0.2) (layer "B.Cu") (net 4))
 (segment (start 42.5 108.7) (end 41.7 109.5) (width 0.2) (layer "B.Cu") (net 4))
 (segment (start 31.2 109) (end 33 109) (width 0.2) (layer "B.Cu") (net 4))
 (segment (start 34 108) (end 42.5 108) (width 0.2) (layer "B.Cu") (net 4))
 (segment (start 33 109) (end 34 108) (width 0.2) (layer "B.Cu") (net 4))
 (segment (start 22.294 126.537186) (end 22.294 133.7365) (width 0.2) (layer "F.Cu") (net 1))
 (segment (start 22.294 143.7585) (end 22.294 152.7865) (width 0.2) (layer "F.Cu") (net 1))
 (segment (start 25.323686 161.6075) (end 22.294 164.637186) (width 0.2) (layer "F.Cu") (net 1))
 (segment (start 72.98375 112.0775) (end 73.81875 112.0775) (width 0.2) (layer "F.Cu") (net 1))
 (segment (start 24.184686 184.5985) (end 25.345314 184.5985) (width 0.2) (layer "F.Cu") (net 1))
 (segment (start 22.294 164.637186) (end 22.294 182.707814) (width 0.2) (layer "F.Cu") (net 1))
 (segment (start 25.323686 123.5075) (end 22.294 126.537186) (width 0.2) (layer "F.Cu") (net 1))
 (segment (start 31.115 142.5575) (end 23.495 142.5575) (width 0.2) (layer "F.Cu") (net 1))
 (segment (start 29.286314 180.6575) (end 31.115 180.6575) (width 0.2) (layer "F.Cu") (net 1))
 (segment (start 31.115 161.6075) (end 25.323686 161.6075) (width 0.2) (layer "F.Cu") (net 1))
 (segment (start 22.294 152.7865) (end 31.115 161.6075) (width 0.2) (layer "F.Cu") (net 1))
 (segment (start 23.495 142.5575) (end 22.294 143.7585) (width 0.2) (layer "F.Cu") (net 1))
 (segment (start 22.294 182.707814) (end 24.184686 184.5985) (width 0.2) (layer "F.Cu") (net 1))
 (segment (start 31.115 123.5075) (end 25.323686 123.5075) (width 0.2) (layer "F.Cu") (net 1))
 (segment (start 25.345314 184.5985) (end 29.286314 180.6575) (width 0.2) (layer "F.Cu") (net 1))
 (segment (start 22.294 133.7365) (end 31.115 142.5575) (width 0.2) (layer "F.Cu") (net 1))
 (segment (start 33.5 110.5) (end 31.2 110.5) (width 0.2) (layer "B.Cu") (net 1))
 (segment (start 36.5 109.5) (end 34.5 109.5) (width 0.2) (layer "B.Cu") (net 1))
 (segment (start 31.115 113.885) (end 34 111) (width 0.2) (layer "B.Cu") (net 1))
 (segment (start 36.1405 113.1405) (end 34 111) (width 0.2) (layer "B.Cu") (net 1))
 (segment (start 72.98375 112.0775) (end 71.92075 113.1405) (width 0.2) (layer "B.Cu") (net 1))
 (segment (start 71.92075 113.1405) (end 36.1405 113.1405) (width 0.2) (layer "B.Cu") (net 1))
 (segment (start 31.115 123.5075) (end 31.115 113.885) (width 0.2) (layer "B.Cu") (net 1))
 (segment (start 34 111) (end 33.5 110.5) (width 0.2) (layer "B.Cu") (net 1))
 (segment (start 34.5 109.5) (end 33.5 110.5) (width 0.2) (layer "B.Cu") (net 1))
 (segment (start 42.696 111) (end 41.7 111) (width 0.2) (layer "B.Cu") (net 3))
 (segment (start 72.94275 109.5375) (end 70.53725 107.132) (width 0.2) (layer "B.Cu") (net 3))
 (segment (start 25.4129 107.132) (end 24.137 108.4079) (width 0.2) (layer "B.Cu") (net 3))
 (segment (start 24.7291 109) (end 24.137 108.4079) (width 0.2) (layer "B.Cu") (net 3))
 (segment (start 71.87975 110.6005) (end 72.94275 109.5375) (width 0.2) (layer "B.Cu") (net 3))
 (segment (start 71.87975 110.6005) (end 43.0955 110.6005) (width 0.2) (layer "B.Cu") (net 3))
 (segment (start 43.0955 110.6005) (end 42.696 111) (width 0.2) (layer "B.Cu") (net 3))
 (segment (start 70.53725 107.132) (end 25.4129 107.132) (width 0.2) (layer "B.Cu") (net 3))
 (segment (start 26 109) (end 24.7291 109) (width 0.2) (layer "B.Cu") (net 3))
 (segment (start 64.09375 126.0475) (end 24.765 126.0475) (width 0.2) (layer "F.Cu") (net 7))
 (segment (start 72.98375 117.1575) (end 64.09375 126.0475) (width 0.2) (layer "F.Cu") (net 7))
 (segment (start 47.58375 145.0975) (end 24.765 145.0975) (width 0.2) (layer "F.Cu") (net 8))
 (segment (start 72.98375 119.6975) (end 47.58375 145.0975) (width 0.2) (layer "F.Cu") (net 8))
 (segment (start 31.07375 164.1475) (end 24.765 164.1475) (width 0.2) (layer "F.Cu") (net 2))
 (segment (start 72.98375 122.2375) (end 31.07375 164.1475) (width 0.2) (layer "F.Cu") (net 2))
 (segment (start 72.98375 124.7775) (end 72.98375 134.97875) (width 0.2) (layer "F.Cu") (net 9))
 (segment (start 72.98375 134.97875) (end 24.765 183.1975) (width 0.2) (layer "F.Cu") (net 9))
 (segment (start 26 110.565) (end 25.78 110.785) (width 0.2) (layer "B.Cu") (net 6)))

